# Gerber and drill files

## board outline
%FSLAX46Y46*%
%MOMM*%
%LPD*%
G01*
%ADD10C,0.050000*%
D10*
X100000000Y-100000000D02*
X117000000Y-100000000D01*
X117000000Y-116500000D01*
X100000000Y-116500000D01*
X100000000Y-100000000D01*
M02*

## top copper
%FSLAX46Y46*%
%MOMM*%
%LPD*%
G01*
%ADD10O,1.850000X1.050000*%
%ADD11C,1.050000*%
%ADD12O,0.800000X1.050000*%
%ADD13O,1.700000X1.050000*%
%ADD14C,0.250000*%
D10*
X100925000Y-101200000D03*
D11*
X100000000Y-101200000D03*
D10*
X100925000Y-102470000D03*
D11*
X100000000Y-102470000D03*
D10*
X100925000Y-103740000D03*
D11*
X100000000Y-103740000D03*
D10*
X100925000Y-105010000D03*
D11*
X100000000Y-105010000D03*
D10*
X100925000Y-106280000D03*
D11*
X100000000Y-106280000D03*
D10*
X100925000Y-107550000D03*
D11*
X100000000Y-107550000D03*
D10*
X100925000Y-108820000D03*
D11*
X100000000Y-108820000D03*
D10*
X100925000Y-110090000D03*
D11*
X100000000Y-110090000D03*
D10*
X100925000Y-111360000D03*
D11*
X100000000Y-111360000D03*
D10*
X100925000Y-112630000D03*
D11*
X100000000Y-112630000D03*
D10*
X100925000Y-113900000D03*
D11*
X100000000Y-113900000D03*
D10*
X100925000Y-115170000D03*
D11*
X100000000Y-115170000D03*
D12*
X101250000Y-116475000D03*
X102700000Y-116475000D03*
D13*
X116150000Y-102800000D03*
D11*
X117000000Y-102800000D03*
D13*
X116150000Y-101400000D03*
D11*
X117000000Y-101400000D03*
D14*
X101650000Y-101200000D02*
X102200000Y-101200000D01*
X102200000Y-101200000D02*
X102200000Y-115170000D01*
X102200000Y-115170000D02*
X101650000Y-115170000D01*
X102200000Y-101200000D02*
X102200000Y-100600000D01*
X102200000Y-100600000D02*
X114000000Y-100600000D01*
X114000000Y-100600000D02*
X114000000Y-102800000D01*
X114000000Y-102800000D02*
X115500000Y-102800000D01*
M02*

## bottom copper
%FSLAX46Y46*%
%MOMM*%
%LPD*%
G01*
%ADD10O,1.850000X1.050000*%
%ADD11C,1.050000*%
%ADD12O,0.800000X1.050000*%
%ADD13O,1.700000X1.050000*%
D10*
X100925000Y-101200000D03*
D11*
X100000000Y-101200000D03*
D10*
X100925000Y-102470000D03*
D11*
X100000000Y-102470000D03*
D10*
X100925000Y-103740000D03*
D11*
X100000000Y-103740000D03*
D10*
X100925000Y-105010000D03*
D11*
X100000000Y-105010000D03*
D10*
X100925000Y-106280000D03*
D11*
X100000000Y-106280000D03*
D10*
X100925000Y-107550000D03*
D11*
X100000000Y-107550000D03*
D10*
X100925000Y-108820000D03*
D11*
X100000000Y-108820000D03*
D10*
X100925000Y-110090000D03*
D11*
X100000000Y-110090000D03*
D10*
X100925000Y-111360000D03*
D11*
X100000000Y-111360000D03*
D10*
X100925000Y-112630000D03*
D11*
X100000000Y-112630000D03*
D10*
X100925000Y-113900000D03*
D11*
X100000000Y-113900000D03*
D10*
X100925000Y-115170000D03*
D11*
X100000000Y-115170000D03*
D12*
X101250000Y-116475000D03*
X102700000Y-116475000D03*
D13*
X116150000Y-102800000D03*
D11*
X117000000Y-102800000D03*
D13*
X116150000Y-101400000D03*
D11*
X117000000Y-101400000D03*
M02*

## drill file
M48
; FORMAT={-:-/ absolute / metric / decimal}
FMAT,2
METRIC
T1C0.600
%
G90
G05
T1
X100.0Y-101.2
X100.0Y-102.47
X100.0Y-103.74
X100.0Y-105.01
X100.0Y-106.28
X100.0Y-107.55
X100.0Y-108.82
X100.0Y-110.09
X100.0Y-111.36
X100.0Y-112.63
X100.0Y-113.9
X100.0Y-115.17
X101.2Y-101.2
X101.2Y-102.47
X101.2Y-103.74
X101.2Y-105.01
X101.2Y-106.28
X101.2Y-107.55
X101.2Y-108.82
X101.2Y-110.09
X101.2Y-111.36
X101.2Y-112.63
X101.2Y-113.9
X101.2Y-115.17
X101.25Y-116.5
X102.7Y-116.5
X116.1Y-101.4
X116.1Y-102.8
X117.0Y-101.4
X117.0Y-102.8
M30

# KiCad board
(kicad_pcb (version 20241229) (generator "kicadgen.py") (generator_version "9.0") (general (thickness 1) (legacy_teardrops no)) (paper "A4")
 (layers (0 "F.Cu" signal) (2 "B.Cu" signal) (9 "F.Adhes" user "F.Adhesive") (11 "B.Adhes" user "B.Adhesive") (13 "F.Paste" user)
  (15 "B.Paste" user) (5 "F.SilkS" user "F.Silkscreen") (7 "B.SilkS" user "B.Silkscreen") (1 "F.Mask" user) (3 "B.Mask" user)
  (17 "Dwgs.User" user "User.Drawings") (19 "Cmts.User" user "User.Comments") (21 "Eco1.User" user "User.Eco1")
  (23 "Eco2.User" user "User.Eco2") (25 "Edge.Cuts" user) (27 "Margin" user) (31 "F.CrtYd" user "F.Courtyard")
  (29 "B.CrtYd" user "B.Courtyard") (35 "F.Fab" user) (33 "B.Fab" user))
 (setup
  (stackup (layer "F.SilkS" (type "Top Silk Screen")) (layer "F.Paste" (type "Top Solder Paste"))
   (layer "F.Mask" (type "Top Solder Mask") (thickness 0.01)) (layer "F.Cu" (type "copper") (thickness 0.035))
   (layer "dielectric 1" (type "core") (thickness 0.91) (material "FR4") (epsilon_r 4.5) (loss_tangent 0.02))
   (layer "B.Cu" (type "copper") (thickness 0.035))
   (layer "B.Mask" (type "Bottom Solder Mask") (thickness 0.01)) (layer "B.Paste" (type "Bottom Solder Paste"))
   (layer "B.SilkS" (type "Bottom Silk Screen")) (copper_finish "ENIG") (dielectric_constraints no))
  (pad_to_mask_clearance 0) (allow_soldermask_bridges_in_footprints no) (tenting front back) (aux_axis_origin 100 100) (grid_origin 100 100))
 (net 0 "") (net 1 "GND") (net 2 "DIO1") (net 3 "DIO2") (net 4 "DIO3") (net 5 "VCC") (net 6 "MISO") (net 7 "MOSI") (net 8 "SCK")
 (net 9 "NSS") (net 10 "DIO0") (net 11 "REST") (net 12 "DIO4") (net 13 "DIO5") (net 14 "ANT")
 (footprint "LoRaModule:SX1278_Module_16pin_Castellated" (layer "F.Cu") (at 100 100)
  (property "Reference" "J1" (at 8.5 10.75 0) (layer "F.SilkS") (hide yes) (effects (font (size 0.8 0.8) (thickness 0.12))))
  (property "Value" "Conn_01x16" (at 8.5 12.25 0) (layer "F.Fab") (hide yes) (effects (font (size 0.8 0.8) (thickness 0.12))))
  (pad "1" thru_hole oval (at 1.2 1.2) (size 1.85 1.05) (drill 0.6 (offset -0.275 0)) (layers "*.Cu" "*.Mask") (remove_unused_layers no)
   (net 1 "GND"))
  (pad "1" thru_hole circle (at 0 1.2) (size 1.05 1.05) (drill 0.6) (layers "*.Cu" "*.Mask") (remove_unused_layers no) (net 1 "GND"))
  (pad "2" thru_hole oval (at 1.2 2.47) (size 1.85 1.05) (drill 0.6 (offset -0.275 0)) (layers "*.Cu" "*.Mask") (remove_unused_layers no)
   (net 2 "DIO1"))
  (pad "2" thru_hole circle (at 0 2.47) (size 1.05 1.05) (drill 0.6) (layers "*.Cu" "*.Mask") (remove_unused_layers no) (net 2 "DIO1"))
  (pad "3" thru_hole oval (at 1.2 3.74) (size 1.85 1.05) (drill 0.6 (offset -0.275 0)) (layers "*.Cu" "*.Mask") (remove_unused_layers no)
   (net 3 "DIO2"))
  (pad "3" thru_hole circle (at 0 3.74) (size 1.05 1.05) (drill 0.6) (layers "*.Cu" "*.Mask") (remove_unused_layers no) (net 3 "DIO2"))
  (pad "4" thru_hole oval (at 1.2 5.01) (size 1.85 1.05) (drill 0.6 (offset -0.275 0)) (layers "*.Cu" "*.Mask") (remove_unused_layers no)
   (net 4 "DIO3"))
  (pad "4" thru_hole circle (at 0 5.01) (size 1.05 1.05) (drill 0.6) (layers "*.Cu" "*.Mask") (remove_unused_layers no) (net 4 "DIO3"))
  (pad "5" thru_hole oval (at 1.2 6.28) (size 1.85 1.05) (drill 0.6 (offset -0.275 0)) (layers "*.Cu" "*.Mask") (remove_unused_layers no)
   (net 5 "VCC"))
  (pad "5" thru_hole circle (at 0 6.28) (size 1.05 1.05) (drill 0.6) (layers "*.Cu" "*.Mask") (remove_unused_layers no) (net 5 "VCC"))
  (pad "6" thru_hole oval (at 1.2 7.55) (size 1.85 1.05) (drill 0.6 (offset -0.275 0)) (layers "*.Cu" "*.Mask") (remove_unused_layers no)
   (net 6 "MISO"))
  (pad "6" thru_hole circle (at 0 7.55) (size 1.05 1.05) (drill 0.6) (layers "*.Cu" "*.Mask") (remove_unused_layers no) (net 6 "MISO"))
  (pad "7" thru_hole oval (at 1.2 8.82) (size 1.85 1.05) (drill 0.6 (offset -0.275 0)) (layers "*.Cu" "*.Mask") (remove_unused_layers no)
   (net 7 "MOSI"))
  (pad "7" thru_hole circle (at 0 8.82) (size 1.05 1.05) (drill 0.6) (layers "*.Cu" "*.Mask") (remove_unused_layers no) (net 7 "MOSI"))
  (pad "8" thru_hole oval (at 1.2 10.09) (size 1.85 1.05) (drill 0.6 (offset -0.275 0)) (layers "*.Cu" "*.Mask") (remove_unused_layers no)
   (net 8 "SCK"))
  (pad "8" thru_hole circle (at 0 10.09) (size 1.05 1.05) (drill 0.6) (layers "*.Cu" "*.Mask") (remove_unused_layers no) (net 8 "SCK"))
  (pad "9" thru_hole oval (at 1.2 11.36) (size 1.85 1.05) (drill 0.6 (offset -0.275 0)) (layers "*.Cu" "*.Mask") (remove_unused_layers no)
   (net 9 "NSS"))
  (pad "9" thru_hole circle (at 0 11.36) (size 1.05 1.05) (drill 0.6) (layers "*.Cu" "*.Mask") (remove_unused_layers no) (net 9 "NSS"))
  (pad "10" thru_hole oval (at 1.2 12.63) (size 1.85 1.05) (drill 0.6 (offset -0.275 0)) (layers "*.Cu" "*.Mask") (remove_unused_layers no)
   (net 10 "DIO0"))
  (pad "10" thru_hole circle (at 0 12.63) (size 1.05 1.05) (drill 0.6) (layers "*.Cu" "*.Mask") (remove_unused_layers no) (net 10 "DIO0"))
  (pad "11" thru_hole oval (at 1.2 13.9) (size 1.85 1.05) (drill 0.6 (offset -0.275 0)) (layers "*.Cu" "*.Mask") (remove_unused_layers no)
   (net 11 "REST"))
  (pad "11" thru_hole circle (at 0 13.9) (size 1.05 1.05) (drill 0.6) (layers "*.Cu" "*.Mask") (remove_unused_layers no) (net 11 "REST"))
  (pad "12" thru_hole oval (at 1.2 15.17) (size 1.85 1.05) (drill 0.6 (offset -0.275 0)) (layers "*.Cu" "*.Mask") (remove_unused_layers no)
   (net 1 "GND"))
  (pad "12" thru_hole circle (at 0 15.17) (size 1.05 1.05) (drill 0.6) (layers "*.Cu" "*.Mask") (remove_unused_layers no) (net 1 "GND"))
  (pad "13" thru_hole oval (at 1.25 16.5) (size 0.8 1.05) (drill 0.6 (offset 0 -0.025)) (layers "*.Cu" "*.Mask") (remove_unused_layers no)
   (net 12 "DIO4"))
  (pad "14" thru_hole oval (at 2.7 16.5) (size 0.8 1.05) (drill 0.6 (offset 0 -0.025)) (layers "*.Cu" "*.Mask") (remove_unused_layers no)
   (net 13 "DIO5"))
  (pad "15" thru_hole oval (at 16.1 2.8) (size 1.7 1.05) (drill 0.6 (offset 0.05 0)) (layers "*.Cu" "*.Mask") (remove_unused_layers no)
   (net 1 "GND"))
  (pad "15" thru_hole circle (at 17 2.8) (size 1.05 1.05) (drill 0.6) (layers "*.Cu" "*.Mask") (remove_unused_layers no) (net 1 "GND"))
  (pad "16" thru_hole oval (at 16.1 1.4) (size 1.7 1.05) (drill 0.6 (offset 0.05 0)) (layers "*.Cu" "*.Mask") (remove_unused_layers no)
   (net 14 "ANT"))
  (pad "16" thru_hole circle (at 17 1.4) (size 1.05 1.05) (drill 0.6) (layers "*.Cu" "*.Mask") (remove_unused_layers no) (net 14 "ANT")))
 (gr_rect (start 100 100) (end 117 116.5) (stroke (width 0.05) (type solid)) (fill no) (layer "Edge.Cuts"))
 (segment (start 101.65 101.2) (end 102.2 101.2) (width 0.25) (layer "F.Cu") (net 1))
 (segment (start 102.2 101.2) (end 102.2 115.17) (width 0.25) (layer "F.Cu") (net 1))
 (segment (start 102.2 115.17) (end 101.65 115.17) (width 0.25) (layer "F.Cu") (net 1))
 (segment (start 102.2 101.2) (end 102.2 100.6) (width 0.25) (layer "F.Cu") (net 1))
 (segment (start 102.2 100.6) (end 114 100.6) (width 0.25) (layer "F.Cu") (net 1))
 (segment (start 114 100.6) (end 114 102.8) (width 0.25) (layer "F.Cu") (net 1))
 (segment (start 114 102.8) (end 115.5 102.8) (width 0.25) (layer "F.Cu") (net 1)))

